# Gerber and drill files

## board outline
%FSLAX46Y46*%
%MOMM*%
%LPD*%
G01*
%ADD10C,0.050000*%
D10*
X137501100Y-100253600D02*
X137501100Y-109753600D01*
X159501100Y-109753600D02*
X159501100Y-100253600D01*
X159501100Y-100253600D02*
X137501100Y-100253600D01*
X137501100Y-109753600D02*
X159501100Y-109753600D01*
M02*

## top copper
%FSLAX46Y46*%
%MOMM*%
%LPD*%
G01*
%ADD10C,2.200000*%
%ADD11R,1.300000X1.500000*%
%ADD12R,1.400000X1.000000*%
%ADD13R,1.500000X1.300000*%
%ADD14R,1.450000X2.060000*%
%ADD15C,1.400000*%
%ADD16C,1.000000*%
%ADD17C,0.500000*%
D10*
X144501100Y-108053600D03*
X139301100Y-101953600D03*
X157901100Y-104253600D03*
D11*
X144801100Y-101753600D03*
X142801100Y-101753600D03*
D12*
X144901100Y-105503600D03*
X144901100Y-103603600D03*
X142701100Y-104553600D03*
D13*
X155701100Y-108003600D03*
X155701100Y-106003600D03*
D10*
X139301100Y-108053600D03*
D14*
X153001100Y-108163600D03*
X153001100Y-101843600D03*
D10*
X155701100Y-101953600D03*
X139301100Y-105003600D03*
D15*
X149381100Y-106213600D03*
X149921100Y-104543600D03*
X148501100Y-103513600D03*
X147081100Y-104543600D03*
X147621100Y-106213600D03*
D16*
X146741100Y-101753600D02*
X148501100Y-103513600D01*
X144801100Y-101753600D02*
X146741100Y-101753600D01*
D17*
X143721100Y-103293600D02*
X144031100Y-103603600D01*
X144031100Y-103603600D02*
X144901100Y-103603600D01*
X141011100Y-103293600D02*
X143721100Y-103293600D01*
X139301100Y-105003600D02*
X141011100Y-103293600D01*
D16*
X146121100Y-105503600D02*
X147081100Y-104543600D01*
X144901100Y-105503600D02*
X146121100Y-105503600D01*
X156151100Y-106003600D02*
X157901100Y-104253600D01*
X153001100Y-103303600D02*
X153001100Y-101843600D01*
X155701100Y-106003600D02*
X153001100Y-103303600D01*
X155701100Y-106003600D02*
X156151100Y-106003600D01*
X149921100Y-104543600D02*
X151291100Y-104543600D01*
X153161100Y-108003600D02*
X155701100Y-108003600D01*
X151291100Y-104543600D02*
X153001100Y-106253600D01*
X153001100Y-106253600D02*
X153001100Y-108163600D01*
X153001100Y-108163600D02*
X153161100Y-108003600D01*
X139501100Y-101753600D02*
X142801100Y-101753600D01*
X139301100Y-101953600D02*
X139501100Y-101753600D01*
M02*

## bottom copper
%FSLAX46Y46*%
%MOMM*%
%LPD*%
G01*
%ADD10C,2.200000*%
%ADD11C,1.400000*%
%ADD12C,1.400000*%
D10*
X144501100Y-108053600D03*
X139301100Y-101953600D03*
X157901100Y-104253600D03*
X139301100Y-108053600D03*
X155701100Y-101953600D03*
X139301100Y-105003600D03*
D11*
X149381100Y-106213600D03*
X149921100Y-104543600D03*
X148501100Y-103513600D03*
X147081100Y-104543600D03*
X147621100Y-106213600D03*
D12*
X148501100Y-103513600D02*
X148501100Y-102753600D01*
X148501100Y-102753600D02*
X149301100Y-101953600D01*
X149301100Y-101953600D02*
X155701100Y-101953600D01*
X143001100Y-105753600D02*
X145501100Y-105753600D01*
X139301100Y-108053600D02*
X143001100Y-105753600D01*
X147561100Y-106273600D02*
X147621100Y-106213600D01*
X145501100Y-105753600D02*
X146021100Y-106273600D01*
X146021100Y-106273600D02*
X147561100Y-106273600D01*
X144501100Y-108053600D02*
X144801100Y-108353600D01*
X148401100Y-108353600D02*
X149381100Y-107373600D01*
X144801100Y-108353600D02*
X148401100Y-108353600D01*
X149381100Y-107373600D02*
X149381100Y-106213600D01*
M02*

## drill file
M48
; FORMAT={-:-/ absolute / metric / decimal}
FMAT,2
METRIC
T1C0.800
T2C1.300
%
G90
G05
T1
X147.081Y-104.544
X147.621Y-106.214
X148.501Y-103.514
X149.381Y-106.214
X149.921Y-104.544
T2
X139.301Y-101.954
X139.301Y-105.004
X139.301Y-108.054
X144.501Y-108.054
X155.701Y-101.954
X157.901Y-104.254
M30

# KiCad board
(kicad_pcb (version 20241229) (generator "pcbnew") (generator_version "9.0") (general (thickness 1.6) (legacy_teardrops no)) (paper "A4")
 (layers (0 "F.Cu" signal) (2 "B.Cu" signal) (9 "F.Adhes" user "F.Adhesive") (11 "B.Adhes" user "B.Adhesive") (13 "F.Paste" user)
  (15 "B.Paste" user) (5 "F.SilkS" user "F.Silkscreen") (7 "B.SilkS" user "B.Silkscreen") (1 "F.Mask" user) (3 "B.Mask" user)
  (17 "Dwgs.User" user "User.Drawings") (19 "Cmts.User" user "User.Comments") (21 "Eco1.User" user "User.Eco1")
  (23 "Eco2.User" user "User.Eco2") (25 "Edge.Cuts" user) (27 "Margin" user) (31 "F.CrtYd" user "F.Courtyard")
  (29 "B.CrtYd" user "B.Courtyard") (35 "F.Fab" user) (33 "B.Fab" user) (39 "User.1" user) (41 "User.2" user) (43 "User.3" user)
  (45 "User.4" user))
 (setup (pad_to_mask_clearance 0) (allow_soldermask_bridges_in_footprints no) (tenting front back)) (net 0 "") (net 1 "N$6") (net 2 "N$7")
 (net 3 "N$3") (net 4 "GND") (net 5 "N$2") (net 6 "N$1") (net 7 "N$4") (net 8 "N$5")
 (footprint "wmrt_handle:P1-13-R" (layer "F.Cu") (at 144.5011 108.0536)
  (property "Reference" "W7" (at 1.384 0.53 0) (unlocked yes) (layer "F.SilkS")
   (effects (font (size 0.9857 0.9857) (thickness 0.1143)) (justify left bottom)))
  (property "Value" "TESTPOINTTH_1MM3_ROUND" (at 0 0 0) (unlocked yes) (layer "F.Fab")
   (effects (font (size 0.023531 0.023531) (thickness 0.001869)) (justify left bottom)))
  (pad "TP" thru_hole circle (at 0 0) (size 2.2 2.2) (drill 1.3) (layers "*.Cu" "*.Mask") (remove_unused_layers no) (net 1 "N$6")
   (solder_mask_margin 0.0508) (thermal_bridge_angle 0)))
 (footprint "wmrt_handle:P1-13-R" (layer "F.Cu") (at 139.3011 101.9536)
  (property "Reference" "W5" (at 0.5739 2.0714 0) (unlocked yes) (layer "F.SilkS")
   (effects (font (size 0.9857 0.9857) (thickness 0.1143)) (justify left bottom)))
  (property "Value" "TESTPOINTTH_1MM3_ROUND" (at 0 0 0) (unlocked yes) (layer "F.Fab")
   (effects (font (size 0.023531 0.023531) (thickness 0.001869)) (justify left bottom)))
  (pad "TP" thru_hole circle (at 0 0) (size 2.2 2.2) (drill 1.3) (layers "*.Cu" "*.Mask") (remove_unused_layers no) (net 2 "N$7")
   (solder_mask_margin 0.0508) (thermal_bridge_angle 0)))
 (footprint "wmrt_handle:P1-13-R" (layer "F.Cu") (at 157.9011 104.2536)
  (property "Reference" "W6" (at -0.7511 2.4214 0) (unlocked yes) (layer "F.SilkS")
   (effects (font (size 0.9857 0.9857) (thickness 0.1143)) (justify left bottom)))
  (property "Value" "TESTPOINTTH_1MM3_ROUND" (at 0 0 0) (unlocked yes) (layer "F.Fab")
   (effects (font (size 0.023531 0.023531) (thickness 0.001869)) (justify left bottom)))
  (pad "TP" thru_hole circle (at 0 0) (size 2.2 2.2) (drill 1.3) (layers "*.Cu" "*.Mask") (remove_unused_layers no) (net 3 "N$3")
   (solder_mask_margin 0.0508) (thermal_bridge_angle 0)))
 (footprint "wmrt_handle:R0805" (layer "F.Cu") (at 143.8011 101.7536 180)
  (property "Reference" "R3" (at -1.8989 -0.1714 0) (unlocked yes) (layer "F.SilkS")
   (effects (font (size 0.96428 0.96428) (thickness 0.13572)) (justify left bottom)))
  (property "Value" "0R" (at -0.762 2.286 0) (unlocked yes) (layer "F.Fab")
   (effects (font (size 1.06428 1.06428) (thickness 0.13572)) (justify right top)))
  (pad "1" smd rect (at -1 0 180) (size 1.3 1.5) (layers "F.Cu" "F.Mask" "F.Paste") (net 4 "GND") (solder_mask_margin 0.0508)
   (solder_paste_margin 0) (thermal_bridge_angle 0))
  (pad "2" smd rect (at 1 0 180) (size 1.3 1.5) (layers "F.Cu" "F.Mask" "F.Paste") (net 2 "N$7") (solder_mask_margin 0.0508)
   (solder_paste_margin 0) (thermal_bridge_angle 0)))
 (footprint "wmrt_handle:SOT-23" (layer "F.Cu") (at 143.8011 104.5536 90)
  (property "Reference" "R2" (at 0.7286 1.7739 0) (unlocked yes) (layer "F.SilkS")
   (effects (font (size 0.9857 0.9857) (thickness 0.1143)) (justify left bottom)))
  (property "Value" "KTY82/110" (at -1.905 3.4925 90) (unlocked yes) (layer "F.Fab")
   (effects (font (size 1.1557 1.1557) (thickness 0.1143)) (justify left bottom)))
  (pad "1" smd rect (at -0.95 1.1 90) (size 1 1.4) (layers "F.Cu" "F.Mask" "F.Paste") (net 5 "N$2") (solder_mask_margin 0.0508)
   (solder_paste_margin 0) (thermal_bridge_angle 0))
  (pad "2" smd rect (at 0.95 1.1 90) (size 1 1.4) (layers "F.Cu" "F.Mask" "F.Paste") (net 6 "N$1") (solder_mask_margin 0.0508)
   (solder_paste_margin 0) (thermal_bridge_angle 0))
  (pad "3" smd rect (at 0 -1.1 90) (size 1 1.4) (layers "F.Cu" "F.Mask" "F.Paste") (solder_mask_margin 0.0508) (solder_paste_margin 0)
   (thermal_bridge_angle 0)))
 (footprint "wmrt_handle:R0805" (layer "F.Cu") (at 155.7011 107.0036 90)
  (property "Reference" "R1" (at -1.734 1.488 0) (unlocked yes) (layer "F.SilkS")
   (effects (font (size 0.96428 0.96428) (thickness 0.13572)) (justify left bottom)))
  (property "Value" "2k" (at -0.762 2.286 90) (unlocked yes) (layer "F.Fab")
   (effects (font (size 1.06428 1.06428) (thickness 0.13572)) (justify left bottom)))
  (pad "1" smd rect (at -1 0 90) (size 1.3 1.5) (layers "F.Cu" "F.Mask" "F.Paste") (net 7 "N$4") (solder_mask_margin 0.0508)
   (solder_paste_margin 0) (thermal_bridge_angle 0))
  (pad "2" smd rect (at 1 0 90) (size 1.3 1.5) (layers "F.Cu" "F.Mask" "F.Paste") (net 3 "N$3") (solder_mask_margin 0.0508)
   (solder_paste_margin 0) (thermal_bridge_angle 0)))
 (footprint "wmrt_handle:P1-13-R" (layer "F.Cu") (at 139.3011 108.0536)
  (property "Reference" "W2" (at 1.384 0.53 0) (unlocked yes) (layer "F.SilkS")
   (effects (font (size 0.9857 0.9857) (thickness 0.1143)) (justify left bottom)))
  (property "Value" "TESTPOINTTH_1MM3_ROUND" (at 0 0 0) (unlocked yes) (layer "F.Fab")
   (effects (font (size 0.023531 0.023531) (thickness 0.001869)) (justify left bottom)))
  (pad "TP" thru_hole circle (at 0 0) (size 2.2 2.2) (drill 1.3) (layers "*.Cu" "*.Mask") (remove_unused_layers no) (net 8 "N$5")
   (solder_mask_margin 0.0508) (thermal_bridge_angle 0)))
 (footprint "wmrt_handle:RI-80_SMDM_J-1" (layer "F.Cu") (at 153.0011 105.0036 90)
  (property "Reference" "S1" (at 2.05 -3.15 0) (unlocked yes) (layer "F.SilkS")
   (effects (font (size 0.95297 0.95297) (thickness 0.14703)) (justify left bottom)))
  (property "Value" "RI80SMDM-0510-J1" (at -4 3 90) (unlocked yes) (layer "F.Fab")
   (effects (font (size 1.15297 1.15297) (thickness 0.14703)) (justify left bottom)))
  (pad "1" smd rect (at -3.16 0 90) (size 2.06 1.45) (layers "F.Cu" "F.Mask" "F.Paste") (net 7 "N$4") (solder_mask_margin 0.0508)
   (solder_paste_margin 0) (thermal_bridge_angle 0))
  (pad "2" smd rect (at 3.16 0 90) (size 2.06 1.45) (layers "F.Cu" "F.Mask" "F.Paste") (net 3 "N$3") (solder_mask_margin 0.0508)
   (solder_paste_margin 0) (thermal_bridge_angle 0)))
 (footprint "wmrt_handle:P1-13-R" (layer "F.Cu") (at 155.7011 101.9536)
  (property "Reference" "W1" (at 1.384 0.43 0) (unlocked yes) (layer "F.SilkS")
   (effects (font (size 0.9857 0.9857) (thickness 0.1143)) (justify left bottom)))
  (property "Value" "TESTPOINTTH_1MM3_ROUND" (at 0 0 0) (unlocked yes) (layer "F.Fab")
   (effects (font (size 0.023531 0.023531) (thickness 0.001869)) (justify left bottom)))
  (pad "TP" thru_hole circle (at 0 0) (size 2.2 2.2) (drill 1.3) (layers "*.Cu" "*.Mask") (remove_unused_layers no) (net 4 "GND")
   (solder_mask_margin 0.0508) (thermal_bridge_angle 0)))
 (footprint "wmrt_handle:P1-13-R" (layer "F.Cu") (at 139.3011 105.0036)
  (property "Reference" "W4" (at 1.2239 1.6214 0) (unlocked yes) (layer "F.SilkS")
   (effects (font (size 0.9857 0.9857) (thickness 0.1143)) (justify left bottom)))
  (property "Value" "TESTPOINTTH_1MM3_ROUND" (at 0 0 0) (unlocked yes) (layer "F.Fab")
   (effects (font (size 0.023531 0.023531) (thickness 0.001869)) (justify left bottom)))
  (pad "TP" thru_hole circle (at 0 0) (size 2.2 2.2) (drill 1.3) (layers "*.Cu" "*.Mask") (remove_unused_layers no) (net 6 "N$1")
   (solder_mask_margin 0.0508) (thermal_bridge_angle 0)))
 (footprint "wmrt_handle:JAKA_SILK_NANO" (layer "B.Cu") (at 154.1311 106.6836 180)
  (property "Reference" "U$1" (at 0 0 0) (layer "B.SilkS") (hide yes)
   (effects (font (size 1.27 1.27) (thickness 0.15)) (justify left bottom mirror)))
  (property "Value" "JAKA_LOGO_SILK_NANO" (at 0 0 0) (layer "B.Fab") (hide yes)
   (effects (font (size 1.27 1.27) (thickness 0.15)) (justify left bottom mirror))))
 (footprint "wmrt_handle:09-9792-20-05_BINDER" (layer "B.Cu") (at 148.5011 105.0036 180)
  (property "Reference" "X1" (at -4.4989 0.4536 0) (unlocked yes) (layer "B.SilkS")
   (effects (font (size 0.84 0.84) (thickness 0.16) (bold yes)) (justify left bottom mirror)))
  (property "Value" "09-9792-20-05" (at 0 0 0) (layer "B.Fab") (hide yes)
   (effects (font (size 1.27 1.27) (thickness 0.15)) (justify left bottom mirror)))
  (pad "1" thru_hole circle (at -0.88 -1.21 180) (size 1.4 1.4) (drill 0.8) (layers "*.Cu" "*.Mask") (remove_unused_layers no) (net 1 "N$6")
   (solder_mask_margin 0.0508) (thermal_bridge_angle 0))
  (pad "2" thru_hole circle (at -1.42 0.46 180) (size 1.4 1.4) (drill 0.8) (layers "*.Cu" "*.Mask") (remove_unused_layers no) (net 7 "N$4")
   (solder_mask_margin 0.0508) (thermal_bridge_angle 0))
  (pad "3" thru_hole circle (at 0 1.49 180) (size 1.4 1.4) (drill 0.8) (layers "*.Cu" "*.Mask") (remove_unused_layers no) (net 4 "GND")
   (solder_mask_margin 0.0508) (thermal_bridge_angle 0))
  (pad "4" thru_hole circle (at 1.42 0.46 180) (size 1.4 1.4) (drill 0.8) (layers "*.Cu" "*.Mask") (remove_unused_layers no) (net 5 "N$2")
   (solder_mask_margin 0.0508) (thermal_bridge_angle 0))
  (pad "5" thru_hole circle (at 0.88 -1.21 180) (size 1.4 1.4) (drill 0.8) (layers "*.Cu" "*.Mask") (remove_unused_layers no) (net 8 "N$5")
   (solder_mask_margin 0.0508) (thermal_bridge_angle 0)))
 (gr_line (start 137.5011 100.2536) (end 137.5011 109.7536) (stroke (width 0.05) (type solid)) (layer "Edge.Cuts"))
 (gr_line (start 159.5011 109.7536) (end 159.5011 100.2536) (stroke (width 0.05) (type solid)) (layer "Edge.Cuts"))
 (gr_line (start 159.5011 100.2536) (end 137.5011 100.2536) (stroke (width 0.05) (type solid)) (layer "Edge.Cuts"))
 (gr_line (start 137.5011 109.7536) (end 159.5011 109.7536) (stroke (width 0.05) (type solid)) (layer "Edge.Cuts"))
 (segment (start 146.7411 101.7536) (end 148.5011 103.5136) (width 1) (layer "F.Cu") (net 4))
 (segment (start 144.8011 101.7536) (end 146.7411 101.7536) (width 1) (layer "F.Cu") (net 4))
 (segment (start 148.5011 103.5136) (end 148.5011 102.7536) (width 1.4) (layer "B.Cu") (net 4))
 (segment (start 148.5011 102.7536) (end 149.3011 101.9536) (width 1.4) (layer "B.Cu") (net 4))
 (segment (start 149.3011 101.9536) (end 155.7011 101.9536) (width 1.4) (layer "B.Cu") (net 4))
 (segment (start 143.7211 103.2936) (end 144.0311 103.6036) (width 0.5) (layer "F.Cu") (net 6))
 (segment (start 144.0311 103.6036) (end 144.9011 103.6036) (width 0.5) (layer "F.Cu") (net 6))
 (segment (start 141.0111 103.2936) (end 143.7211 103.2936) (width 0.5) (layer "F.Cu") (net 6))
 (segment (start 139.3011 105.0036) (end 141.0111 103.2936) (width 0.5) (layer "F.Cu") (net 6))
 (segment (start 146.1211 105.5036) (end 147.0811 104.5436) (width 1) (layer "F.Cu") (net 5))
 (segment (start 144.9011 105.5036) (end 146.1211 105.5036) (width 1) (layer "F.Cu") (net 5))
 (segment (start 156.1511 106.0036) (end 157.9011 104.2536) (width 1) (layer "F.Cu") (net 3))
 (segment (start 153.0011 103.3036) (end 153.0011 101.8436) (width 1) (layer "F.Cu") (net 3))
 (segment (start 155.7011 106.0036) (end 153.0011 103.3036) (width 1) (layer "F.Cu") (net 3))
 (segment (start 155.7011 106.0036) (end 156.1511 106.0036) (width 1) (layer "F.Cu") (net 3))
 (segment (start 149.9211 104.5436) (end 151.2911 104.5436) (width 1) (layer "F.Cu") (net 7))
 (segment (start 153.1611 108.0036) (end 155.7011 108.0036) (width 1) (layer "F.Cu") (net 7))
 (segment (start 151.2911 104.5436) (end 153.0011 106.2536) (width 1) (layer "F.Cu") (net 7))
 (segment (start 153.0011 106.2536) (end 153.0011 108.1636) (width 1) (layer "F.Cu") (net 7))
 (segment (start 153.0011 108.1636) (end 153.1611 108.0036) (width 1) (layer "F.Cu") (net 7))
 (segment (start 143.0011 105.7536) (end 145.5011 105.7536) (width 1.4) (layer "B.Cu") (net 8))
 (segment (start 139.3011 108.0536) (end 143.0011 105.7536) (width 1.4) (layer "B.Cu") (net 8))
 (segment (start 147.5611 106.2736) (end 147.6211 106.2136) (width 1.4) (layer "B.Cu") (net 8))
 (segment (start 145.5011 105.7536) (end 146.0211 106.2736) (width 1.4) (layer "B.Cu") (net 8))
 (segment (start 146.0211 106.2736) (end 147.5611 106.2736) (width 1.4) (layer "B.Cu") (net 8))
 (segment (start 144.5011 108.0536) (end 144.8011 108.3536) (width 1.4) (layer "B.Cu") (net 1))
 (segment (start 148.4011 108.3536) (end 149.3811 107.3736) (width 1.4) (layer "B.Cu") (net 1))
 (segment (start 144.8011 108.3536) (end 148.4011 108.3536) (width 1.4) (layer "B.Cu") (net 1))
 (segment (start 149.3811 107.3736) (end 149.3811 106.2136) (width 1.4) (layer "B.Cu") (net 1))
 (segment (start 139.5011 101.7536) (end 142.8011 101.7536) (width 1) (layer "F.Cu") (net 2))
 (segment (start 139.3011 101.9536) (end 139.5011 101.7536) (width 1) (layer "F.Cu") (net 2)))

